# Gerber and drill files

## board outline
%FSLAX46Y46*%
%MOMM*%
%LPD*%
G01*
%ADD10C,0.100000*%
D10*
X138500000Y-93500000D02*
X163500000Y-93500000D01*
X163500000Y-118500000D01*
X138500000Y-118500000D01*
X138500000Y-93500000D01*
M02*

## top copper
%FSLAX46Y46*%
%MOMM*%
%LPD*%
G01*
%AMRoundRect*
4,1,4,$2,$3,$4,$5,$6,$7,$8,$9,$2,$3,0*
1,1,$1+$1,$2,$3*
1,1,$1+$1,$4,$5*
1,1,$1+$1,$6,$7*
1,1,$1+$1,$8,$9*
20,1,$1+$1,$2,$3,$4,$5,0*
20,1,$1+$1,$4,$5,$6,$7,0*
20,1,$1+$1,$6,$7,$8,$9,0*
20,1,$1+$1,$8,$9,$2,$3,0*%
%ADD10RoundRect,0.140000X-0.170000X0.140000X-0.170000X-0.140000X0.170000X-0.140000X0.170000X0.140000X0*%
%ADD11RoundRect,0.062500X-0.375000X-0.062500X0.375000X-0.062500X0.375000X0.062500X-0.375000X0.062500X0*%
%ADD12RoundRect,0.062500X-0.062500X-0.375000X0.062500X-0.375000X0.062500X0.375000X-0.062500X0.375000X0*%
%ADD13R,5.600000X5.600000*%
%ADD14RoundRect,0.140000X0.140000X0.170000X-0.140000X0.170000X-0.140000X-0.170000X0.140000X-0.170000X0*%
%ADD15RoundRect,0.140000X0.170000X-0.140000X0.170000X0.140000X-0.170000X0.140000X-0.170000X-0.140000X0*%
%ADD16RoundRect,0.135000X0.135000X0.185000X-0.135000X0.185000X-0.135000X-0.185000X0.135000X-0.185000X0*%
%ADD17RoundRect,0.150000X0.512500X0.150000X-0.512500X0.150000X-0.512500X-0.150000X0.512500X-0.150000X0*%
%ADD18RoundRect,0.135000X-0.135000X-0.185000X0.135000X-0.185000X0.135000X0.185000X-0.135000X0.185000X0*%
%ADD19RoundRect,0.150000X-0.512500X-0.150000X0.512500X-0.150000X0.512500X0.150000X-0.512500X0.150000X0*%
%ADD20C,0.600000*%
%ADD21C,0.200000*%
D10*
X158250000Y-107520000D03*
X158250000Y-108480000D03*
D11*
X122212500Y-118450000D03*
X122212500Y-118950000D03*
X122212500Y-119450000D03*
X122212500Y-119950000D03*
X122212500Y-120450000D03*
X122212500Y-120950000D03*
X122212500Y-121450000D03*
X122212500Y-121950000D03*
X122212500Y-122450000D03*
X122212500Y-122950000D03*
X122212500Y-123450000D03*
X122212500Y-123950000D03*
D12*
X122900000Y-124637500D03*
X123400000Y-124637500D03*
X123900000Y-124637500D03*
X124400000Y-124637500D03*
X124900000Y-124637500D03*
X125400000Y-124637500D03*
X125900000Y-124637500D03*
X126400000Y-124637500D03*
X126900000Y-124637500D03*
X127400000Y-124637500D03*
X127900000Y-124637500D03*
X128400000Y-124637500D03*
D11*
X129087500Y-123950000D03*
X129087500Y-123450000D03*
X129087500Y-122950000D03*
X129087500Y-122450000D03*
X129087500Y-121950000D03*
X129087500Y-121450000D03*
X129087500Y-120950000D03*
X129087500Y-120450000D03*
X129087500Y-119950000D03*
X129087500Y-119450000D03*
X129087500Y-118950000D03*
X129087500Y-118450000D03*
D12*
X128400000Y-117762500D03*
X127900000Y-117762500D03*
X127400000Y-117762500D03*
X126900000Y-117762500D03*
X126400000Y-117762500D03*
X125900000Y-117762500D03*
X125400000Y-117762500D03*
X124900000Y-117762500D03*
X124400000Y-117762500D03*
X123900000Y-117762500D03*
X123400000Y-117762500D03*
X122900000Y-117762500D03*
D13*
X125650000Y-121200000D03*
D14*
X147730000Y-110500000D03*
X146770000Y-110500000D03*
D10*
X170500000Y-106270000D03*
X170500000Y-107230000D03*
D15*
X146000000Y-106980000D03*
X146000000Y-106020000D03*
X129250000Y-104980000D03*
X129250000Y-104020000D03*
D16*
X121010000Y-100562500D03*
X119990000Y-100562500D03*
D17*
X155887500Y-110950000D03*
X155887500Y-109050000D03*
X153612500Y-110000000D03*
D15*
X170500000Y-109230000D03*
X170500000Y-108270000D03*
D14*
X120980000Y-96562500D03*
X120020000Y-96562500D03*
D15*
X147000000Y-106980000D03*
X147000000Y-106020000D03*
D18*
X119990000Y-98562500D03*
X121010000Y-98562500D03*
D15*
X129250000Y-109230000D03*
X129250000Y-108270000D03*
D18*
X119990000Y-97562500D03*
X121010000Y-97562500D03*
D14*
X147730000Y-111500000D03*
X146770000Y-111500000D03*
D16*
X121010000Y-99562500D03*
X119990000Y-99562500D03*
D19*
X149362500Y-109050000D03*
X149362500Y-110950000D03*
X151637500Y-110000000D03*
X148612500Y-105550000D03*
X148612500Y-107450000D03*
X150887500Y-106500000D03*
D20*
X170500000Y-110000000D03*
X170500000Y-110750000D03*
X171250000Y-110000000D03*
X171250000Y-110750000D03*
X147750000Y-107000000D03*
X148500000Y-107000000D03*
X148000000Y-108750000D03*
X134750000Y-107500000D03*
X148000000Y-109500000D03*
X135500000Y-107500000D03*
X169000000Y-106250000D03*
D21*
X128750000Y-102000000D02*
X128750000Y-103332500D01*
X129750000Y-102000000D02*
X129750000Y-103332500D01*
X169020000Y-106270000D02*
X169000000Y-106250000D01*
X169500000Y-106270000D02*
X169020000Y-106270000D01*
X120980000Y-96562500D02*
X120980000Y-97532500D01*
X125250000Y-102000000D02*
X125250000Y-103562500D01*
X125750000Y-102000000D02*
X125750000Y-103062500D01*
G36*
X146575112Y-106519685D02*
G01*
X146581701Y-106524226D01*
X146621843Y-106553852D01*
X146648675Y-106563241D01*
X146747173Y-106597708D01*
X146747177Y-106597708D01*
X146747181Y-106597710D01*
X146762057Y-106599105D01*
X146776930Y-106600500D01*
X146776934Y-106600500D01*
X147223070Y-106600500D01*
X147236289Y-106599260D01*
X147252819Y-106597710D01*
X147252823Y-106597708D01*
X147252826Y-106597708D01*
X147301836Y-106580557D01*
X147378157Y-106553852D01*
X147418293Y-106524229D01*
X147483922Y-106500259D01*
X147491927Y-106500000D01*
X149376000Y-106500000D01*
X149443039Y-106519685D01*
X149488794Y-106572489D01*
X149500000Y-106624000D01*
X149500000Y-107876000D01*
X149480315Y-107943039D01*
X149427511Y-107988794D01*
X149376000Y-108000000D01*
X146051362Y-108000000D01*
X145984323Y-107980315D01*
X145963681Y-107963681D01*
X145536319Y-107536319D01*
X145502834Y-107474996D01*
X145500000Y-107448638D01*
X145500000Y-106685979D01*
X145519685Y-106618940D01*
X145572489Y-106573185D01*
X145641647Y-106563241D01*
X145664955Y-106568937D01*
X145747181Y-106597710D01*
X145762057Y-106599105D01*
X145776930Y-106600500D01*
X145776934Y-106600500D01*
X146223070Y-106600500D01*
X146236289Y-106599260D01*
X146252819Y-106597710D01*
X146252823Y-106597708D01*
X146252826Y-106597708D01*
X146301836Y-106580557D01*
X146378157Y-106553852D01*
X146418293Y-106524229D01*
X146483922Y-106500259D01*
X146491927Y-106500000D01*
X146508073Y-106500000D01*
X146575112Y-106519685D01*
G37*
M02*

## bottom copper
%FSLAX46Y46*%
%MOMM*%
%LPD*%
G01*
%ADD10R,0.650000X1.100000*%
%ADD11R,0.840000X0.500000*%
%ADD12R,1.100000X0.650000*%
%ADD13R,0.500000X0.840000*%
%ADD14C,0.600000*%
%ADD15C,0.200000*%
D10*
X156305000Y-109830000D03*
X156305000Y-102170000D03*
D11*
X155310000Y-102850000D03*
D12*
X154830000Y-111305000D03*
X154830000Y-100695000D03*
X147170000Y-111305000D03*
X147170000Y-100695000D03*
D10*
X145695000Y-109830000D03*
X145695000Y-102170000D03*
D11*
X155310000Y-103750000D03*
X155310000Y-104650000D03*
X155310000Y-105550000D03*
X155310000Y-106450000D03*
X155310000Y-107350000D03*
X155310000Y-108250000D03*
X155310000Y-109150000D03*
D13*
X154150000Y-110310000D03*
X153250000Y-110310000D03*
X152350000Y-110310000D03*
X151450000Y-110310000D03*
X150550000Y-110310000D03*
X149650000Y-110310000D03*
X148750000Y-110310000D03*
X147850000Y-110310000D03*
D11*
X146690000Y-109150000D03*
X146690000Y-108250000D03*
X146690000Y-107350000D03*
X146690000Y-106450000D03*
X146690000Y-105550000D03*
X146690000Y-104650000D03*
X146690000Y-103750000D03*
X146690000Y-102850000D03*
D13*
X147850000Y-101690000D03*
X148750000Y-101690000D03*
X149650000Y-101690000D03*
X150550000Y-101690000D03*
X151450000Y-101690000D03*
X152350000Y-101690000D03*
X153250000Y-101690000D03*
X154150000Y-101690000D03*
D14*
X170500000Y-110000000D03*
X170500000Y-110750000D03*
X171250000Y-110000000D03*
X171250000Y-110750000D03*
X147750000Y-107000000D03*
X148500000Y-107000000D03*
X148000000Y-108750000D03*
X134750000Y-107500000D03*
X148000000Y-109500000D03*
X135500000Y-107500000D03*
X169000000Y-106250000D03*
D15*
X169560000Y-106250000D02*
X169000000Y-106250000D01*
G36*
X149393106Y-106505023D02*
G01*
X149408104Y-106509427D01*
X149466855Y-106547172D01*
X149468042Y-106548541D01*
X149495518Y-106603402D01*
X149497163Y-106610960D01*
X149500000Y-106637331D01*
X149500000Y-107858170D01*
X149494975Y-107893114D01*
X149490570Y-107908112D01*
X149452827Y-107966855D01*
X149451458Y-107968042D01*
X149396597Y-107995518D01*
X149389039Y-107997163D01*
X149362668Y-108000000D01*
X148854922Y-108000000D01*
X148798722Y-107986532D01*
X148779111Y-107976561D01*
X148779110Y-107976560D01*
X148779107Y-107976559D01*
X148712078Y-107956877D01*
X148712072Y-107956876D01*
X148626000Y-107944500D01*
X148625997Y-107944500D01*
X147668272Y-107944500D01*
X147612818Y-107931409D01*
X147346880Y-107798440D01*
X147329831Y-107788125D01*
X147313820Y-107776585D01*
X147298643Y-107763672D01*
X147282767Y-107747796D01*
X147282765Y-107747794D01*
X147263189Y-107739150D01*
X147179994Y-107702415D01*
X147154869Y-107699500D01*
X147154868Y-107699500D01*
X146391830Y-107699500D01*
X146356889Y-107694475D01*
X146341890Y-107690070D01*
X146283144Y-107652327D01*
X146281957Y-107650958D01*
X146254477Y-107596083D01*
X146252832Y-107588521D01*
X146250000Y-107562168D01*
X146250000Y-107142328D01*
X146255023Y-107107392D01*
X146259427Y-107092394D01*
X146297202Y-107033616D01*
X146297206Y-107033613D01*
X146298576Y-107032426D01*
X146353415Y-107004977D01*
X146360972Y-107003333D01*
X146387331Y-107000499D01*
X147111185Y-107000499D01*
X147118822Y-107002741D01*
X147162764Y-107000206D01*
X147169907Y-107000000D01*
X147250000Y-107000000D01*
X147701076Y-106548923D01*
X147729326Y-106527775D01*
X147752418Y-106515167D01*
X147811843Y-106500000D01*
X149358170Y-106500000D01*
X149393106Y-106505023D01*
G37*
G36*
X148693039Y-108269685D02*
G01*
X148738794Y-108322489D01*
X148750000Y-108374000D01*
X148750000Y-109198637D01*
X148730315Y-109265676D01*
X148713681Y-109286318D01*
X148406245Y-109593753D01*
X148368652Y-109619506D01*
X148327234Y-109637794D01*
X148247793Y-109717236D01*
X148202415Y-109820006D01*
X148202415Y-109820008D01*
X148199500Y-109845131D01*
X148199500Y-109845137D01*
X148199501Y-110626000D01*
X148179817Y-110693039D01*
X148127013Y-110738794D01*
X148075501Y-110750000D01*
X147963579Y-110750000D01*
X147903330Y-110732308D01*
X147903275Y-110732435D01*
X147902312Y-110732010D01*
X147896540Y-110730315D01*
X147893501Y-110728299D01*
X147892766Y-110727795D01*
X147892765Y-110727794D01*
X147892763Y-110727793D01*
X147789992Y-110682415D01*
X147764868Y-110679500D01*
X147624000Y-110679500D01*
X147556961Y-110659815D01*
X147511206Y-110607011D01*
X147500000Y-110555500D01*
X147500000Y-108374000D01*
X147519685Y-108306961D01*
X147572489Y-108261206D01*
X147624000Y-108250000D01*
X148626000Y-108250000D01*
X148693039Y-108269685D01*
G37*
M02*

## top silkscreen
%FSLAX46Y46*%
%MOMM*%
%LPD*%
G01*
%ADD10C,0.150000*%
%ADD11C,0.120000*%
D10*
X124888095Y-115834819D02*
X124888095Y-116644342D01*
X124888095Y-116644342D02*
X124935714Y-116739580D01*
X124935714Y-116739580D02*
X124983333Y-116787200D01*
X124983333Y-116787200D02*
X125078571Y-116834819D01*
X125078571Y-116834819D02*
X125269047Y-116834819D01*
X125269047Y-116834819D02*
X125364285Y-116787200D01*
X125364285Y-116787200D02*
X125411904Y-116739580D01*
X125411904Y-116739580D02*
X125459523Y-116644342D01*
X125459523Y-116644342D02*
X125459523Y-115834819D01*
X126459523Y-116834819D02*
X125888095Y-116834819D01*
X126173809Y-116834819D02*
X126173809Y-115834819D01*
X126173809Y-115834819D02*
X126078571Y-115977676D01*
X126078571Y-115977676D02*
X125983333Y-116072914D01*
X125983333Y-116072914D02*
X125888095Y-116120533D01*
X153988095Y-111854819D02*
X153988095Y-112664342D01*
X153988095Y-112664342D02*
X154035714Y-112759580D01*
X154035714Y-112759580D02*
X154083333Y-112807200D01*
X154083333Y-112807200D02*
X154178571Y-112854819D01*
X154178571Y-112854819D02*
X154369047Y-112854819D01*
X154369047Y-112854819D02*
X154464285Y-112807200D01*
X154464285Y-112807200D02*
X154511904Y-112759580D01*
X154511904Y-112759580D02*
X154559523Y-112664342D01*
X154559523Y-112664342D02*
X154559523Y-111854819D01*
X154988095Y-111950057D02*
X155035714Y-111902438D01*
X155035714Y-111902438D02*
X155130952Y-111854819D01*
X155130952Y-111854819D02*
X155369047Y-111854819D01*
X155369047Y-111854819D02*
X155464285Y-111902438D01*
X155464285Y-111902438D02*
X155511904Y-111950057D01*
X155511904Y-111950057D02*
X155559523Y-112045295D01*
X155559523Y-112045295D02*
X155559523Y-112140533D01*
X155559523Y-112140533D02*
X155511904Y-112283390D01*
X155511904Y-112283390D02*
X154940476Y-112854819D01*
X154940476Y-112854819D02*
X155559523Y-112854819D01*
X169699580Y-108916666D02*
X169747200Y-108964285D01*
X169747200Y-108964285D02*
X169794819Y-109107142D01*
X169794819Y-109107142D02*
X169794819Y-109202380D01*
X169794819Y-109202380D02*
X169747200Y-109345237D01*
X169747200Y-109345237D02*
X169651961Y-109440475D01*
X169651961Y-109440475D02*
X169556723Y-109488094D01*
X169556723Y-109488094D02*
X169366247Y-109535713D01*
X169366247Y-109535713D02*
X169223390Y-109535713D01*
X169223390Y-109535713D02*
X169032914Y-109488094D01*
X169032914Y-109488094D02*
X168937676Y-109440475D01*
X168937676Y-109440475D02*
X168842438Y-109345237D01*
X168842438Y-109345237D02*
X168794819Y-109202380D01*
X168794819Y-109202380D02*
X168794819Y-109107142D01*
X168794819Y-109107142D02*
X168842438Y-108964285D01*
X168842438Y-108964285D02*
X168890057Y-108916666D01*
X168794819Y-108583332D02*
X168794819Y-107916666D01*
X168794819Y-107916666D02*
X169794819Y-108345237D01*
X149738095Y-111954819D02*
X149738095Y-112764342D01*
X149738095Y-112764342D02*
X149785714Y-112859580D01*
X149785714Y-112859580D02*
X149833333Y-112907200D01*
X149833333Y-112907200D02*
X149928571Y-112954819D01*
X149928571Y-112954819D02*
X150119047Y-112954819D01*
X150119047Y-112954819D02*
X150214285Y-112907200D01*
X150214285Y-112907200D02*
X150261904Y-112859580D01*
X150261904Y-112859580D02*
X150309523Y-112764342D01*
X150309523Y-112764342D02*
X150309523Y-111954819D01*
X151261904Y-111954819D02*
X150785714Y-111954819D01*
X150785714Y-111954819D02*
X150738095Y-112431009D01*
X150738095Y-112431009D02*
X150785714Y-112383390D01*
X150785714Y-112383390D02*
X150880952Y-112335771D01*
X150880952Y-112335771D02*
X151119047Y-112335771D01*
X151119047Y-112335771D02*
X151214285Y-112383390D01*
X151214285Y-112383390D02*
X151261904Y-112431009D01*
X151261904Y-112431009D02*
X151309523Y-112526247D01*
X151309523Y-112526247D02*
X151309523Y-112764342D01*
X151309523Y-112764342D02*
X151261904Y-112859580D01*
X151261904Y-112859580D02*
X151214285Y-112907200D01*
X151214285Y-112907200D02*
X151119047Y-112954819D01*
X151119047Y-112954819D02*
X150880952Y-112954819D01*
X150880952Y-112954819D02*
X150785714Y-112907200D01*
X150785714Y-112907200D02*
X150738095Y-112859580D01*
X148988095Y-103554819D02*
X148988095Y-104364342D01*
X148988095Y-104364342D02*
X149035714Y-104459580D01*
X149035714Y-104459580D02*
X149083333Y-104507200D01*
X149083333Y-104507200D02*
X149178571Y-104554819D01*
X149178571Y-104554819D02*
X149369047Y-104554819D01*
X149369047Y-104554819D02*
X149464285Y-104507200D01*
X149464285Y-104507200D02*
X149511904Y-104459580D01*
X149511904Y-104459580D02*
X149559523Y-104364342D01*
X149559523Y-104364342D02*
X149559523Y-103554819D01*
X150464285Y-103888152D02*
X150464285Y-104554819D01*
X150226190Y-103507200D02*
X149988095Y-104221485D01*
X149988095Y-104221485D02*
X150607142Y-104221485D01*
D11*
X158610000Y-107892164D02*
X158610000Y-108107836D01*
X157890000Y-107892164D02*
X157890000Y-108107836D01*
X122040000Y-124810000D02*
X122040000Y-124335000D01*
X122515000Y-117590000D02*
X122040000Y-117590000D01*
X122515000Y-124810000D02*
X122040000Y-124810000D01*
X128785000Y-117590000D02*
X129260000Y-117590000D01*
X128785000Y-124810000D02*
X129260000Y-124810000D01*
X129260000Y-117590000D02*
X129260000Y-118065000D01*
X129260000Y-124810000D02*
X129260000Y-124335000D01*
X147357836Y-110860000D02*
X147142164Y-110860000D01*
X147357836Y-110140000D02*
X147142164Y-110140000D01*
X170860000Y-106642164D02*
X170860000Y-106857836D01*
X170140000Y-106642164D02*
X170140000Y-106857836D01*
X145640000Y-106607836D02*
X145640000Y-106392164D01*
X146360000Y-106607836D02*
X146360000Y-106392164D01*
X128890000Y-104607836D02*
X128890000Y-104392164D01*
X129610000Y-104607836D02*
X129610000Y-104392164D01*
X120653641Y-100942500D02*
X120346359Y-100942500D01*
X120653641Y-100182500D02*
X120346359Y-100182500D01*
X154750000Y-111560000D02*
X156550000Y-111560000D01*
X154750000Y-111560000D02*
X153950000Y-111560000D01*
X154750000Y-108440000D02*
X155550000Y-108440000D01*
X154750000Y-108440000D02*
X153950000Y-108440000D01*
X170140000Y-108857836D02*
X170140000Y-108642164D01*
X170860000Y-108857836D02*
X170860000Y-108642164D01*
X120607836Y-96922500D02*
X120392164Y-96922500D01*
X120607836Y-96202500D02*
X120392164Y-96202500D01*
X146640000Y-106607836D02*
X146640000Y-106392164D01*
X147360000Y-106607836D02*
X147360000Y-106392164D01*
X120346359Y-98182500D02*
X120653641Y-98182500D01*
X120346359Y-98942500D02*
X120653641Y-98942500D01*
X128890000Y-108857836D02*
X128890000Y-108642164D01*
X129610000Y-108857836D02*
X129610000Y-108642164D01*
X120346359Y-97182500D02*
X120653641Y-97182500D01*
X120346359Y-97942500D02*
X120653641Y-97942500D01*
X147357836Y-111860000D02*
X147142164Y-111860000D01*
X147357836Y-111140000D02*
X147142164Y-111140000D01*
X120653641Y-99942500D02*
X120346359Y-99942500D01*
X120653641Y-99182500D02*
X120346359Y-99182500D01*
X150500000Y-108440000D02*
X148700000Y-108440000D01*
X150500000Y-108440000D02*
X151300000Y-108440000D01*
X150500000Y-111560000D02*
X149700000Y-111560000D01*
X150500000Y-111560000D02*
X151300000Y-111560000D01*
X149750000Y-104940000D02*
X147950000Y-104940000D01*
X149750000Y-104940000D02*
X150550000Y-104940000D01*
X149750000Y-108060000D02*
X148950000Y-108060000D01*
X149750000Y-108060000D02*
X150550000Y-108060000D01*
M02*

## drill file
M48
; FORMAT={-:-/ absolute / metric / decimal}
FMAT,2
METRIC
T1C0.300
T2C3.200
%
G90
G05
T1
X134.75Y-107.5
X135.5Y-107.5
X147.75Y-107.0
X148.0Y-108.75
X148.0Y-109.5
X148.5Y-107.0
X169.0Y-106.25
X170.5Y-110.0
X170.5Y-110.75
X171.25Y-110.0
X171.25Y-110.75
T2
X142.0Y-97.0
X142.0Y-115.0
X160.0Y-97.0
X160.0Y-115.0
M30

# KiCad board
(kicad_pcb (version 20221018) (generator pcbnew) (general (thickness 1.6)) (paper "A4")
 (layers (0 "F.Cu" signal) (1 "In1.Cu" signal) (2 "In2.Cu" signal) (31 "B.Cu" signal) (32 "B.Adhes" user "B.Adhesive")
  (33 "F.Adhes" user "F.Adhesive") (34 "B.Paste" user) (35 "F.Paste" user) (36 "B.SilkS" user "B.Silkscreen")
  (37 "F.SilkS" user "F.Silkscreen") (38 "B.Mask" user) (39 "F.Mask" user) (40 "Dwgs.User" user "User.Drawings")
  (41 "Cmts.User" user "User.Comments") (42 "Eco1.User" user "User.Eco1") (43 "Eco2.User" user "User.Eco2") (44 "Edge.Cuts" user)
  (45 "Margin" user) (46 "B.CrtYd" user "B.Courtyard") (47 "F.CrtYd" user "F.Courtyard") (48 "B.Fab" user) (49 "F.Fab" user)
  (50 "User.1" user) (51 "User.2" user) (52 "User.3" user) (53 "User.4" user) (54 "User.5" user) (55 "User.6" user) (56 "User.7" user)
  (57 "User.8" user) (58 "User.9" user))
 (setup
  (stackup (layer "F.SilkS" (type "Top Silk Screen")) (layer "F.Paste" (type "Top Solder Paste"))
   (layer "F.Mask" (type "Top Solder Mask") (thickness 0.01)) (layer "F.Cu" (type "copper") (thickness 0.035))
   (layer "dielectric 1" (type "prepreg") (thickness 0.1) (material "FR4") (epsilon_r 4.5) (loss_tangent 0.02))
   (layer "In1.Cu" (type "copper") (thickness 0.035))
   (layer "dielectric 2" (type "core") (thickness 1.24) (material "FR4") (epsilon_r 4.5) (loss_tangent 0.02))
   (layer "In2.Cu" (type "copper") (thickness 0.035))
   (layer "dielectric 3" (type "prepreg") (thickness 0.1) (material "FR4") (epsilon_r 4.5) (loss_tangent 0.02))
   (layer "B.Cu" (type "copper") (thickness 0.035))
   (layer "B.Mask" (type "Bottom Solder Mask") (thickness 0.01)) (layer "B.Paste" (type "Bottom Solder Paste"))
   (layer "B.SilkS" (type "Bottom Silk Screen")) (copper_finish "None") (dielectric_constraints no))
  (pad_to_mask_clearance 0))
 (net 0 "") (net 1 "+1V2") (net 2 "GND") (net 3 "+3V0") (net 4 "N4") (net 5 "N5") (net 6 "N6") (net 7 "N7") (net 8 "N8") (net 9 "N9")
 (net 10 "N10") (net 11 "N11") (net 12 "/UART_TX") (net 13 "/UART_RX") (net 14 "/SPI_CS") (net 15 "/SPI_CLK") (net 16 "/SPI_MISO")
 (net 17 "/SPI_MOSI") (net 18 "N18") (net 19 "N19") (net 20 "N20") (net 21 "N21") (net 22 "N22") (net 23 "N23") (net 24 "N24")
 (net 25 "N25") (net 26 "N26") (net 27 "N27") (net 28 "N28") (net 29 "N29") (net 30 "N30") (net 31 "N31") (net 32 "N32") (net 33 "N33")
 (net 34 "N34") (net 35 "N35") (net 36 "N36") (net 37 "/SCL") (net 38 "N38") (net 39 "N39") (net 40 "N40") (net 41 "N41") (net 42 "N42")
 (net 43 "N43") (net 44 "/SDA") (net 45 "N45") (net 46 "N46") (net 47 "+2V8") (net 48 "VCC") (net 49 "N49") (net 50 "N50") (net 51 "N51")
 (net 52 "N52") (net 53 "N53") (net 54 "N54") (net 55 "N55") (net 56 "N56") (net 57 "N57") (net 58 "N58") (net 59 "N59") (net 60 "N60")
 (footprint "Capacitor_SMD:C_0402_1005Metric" (layer "F.Cu") (at 158.25 108 -90)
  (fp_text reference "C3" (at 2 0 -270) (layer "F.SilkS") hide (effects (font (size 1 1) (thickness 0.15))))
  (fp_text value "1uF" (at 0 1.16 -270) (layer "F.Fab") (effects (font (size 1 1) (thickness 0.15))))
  (fp_line (start -0.107836 -0.36) (end 0.107836 -0.36) (stroke (width 0.12) (type solid)) (layer "F.SilkS"))
  (fp_line (start -0.107836 0.36) (end 0.107836 0.36) (stroke (width 0.12) (type solid)) (layer "F.SilkS"))
  (pad "1" smd roundrect (at -0.48 0 270) (size 0.56 0.62) (layers "F.Cu" "F.Paste" "F.Mask") (roundrect_rratio 0.25) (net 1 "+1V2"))
  (pad "2" smd roundrect (at 0.48 0 270) (size 0.56 0.62) (layers "F.Cu" "F.Paste" "F.Mask") (roundrect_rratio 0.25) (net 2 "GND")))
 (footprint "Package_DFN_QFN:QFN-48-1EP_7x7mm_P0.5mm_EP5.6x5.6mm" (layer "F.Cu") (at 125.65 121.2)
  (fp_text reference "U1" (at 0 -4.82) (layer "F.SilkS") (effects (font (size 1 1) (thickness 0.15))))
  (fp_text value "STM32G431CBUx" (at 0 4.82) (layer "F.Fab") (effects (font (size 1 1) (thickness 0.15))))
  (fp_line (start -3.61 3.61) (end -3.61 3.135) (stroke (width 0.12) (type solid)) (layer "F.SilkS"))
  (fp_line (start -3.135 -3.61) (end -3.61 -3.61) (stroke (width 0.12) (type solid)) (layer "F.SilkS"))
  (fp_line (start -3.135 3.61) (end -3.61 3.61) (stroke (width 0.12) (type solid)) (layer "F.SilkS"))
  (fp_line (start 3.135 -3.61) (end 3.61 -3.61) (stroke (width 0.12) (type solid)) (layer "F.SilkS"))
  (fp_line (start 3.135 3.61) (end 3.61 3.61) (stroke (width 0.12) (type solid)) (layer "F.SilkS"))
  (fp_line (start 3.61 -3.61) (end 3.61 -3.135) (stroke (width 0.12) (type solid)) (layer "F.SilkS"))
  (fp_line (start 3.61 3.61) (end 3.61 3.135) (stroke (width 0.12) (type solid)) (layer "F.SilkS"))
  (pad "" smd roundrect (at -2.1 -2.1) (size 1.13 1.13) (layers "F.Paste") (roundrect_rratio 0.221239))
  (pad "" smd roundrect (at -2.1 -0.7) (size 1.13 1.13) (layers "F.Paste") (roundrect_rratio 0.221239))
  (pad "" smd roundrect (at -2.1 0.7) (size 1.13 1.13) (layers "F.Paste") (roundrect_rratio 0.221239))
  (pad "" smd roundrect (at -2.1 2.1) (size 1.13 1.13) (layers "F.Paste") (roundrect_rratio 0.221239))
  (pad "" smd roundrect (at -0.7 -2.1) (size 1.13 1.13) (layers "F.Paste") (roundrect_rratio 0.221239))
  (pad "" smd roundrect (at -0.7 -0.7) (size 1.13 1.13) (layers "F.Paste") (roundrect_rratio 0.221239))
  (pad "" smd roundrect (at -0.7 0.7) (size 1.13 1.13) (layers "F.Paste") (roundrect_rratio 0.221239))
  (pad "" smd roundrect (at -0.7 2.1) (size 1.13 1.13) (layers "F.Paste") (roundrect_rratio 0.221239))
  (pad "" smd roundrect (at 0.7 -2.1) (size 1.13 1.13) (layers "F.Paste") (roundrect_rratio 0.221239))
  (pad "" smd roundrect (at 0.7 -0.7) (size 1.13 1.13) (layers "F.Paste") (roundrect_rratio 0.221239))
  (pad "" smd roundrect (at 0.7 0.7) (size 1.13 1.13) (layers "F.Paste") (roundrect_rratio 0.221239))
  (pad "" smd roundrect (at 0.7 2.1) (size 1.13 1.13) (layers "F.Paste") (roundrect_rratio 0.221239))
  (pad "" smd roundrect (at 2.1 -2.1) (size 1.13 1.13) (layers "F.Paste") (roundrect_rratio 0.221239))
  (pad "" smd roundrect (at 2.1 -0.7) (size 1.13 1.13) (layers "F.Paste") (roundrect_rratio 0.221239))
  (pad "" smd roundrect (at 2.1 0.7) (size 1.13 1.13) (layers "F.Paste") (roundrect_rratio 0.221239))
  (pad "" smd roundrect (at 2.1 2.1) (size 1.13 1.13) (layers "F.Paste") (roundrect_rratio 0.221239))
  (pad "1" smd roundrect (at -3.4375 -2.75) (size 0.875 0.25) (layers "F.Cu" "F.Paste" "F.Mask") (roundrect_rratio 0.25) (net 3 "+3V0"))
  (pad "2" smd roundrect (at -3.4375 -2.25) (size 0.875 0.25) (layers "F.Cu" "F.Paste" "F.Mask") (roundrect_rratio 0.25) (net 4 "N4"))
  (pad "3" smd roundrect (at -3.4375 -1.75) (size 0.875 0.25) (layers "F.Cu" "F.Paste" "F.Mask") (roundrect_rratio 0.25) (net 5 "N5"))
  (pad "4" smd roundrect (at -3.4375 -1.25) (size 0.875 0.25) (layers "F.Cu" "F.Paste" "F.Mask") (roundrect_rratio 0.25) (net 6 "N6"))
  (pad "5" smd roundrect (at -3.4375 -0.75) (size 0.875 0.25) (layers "F.Cu" "F.Paste" "F.Mask") (roundrect_rratio 0.25) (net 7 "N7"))
  (pad "6" smd roundrect (at -3.4375 -0.25) (size 0.875 0.25) (layers "F.Cu" "F.Paste" "F.Mask") (roundrect_rratio 0.25) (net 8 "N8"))
  (pad "7" smd roundrect (at -3.4375 0.25) (size 0.875 0.25) (layers "F.Cu" "F.Paste" "F.Mask") (roundrect_rratio 0.25) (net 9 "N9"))
  (pad "8" smd roundrect (at -3.4375 0.75) (size 0.875 0.25) (layers "F.Cu" "F.Paste" "F.Mask") (roundrect_rratio 0.25) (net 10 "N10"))
  (pad "9" smd roundrect (at -3.4375 1.25) (size 0.875 0.25) (layers "F.Cu" "F.Paste" "F.Mask") (roundrect_rratio 0.25) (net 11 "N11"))
  (pad "10" smd roundrect (at -3.4375 1.75) (size 0.875 0.25) (layers "F.Cu" "F.Paste" "F.Mask") (roundrect_rratio 0.25) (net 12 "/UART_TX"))
  (pad "11" smd roundrect (at -3.4375 2.25) (size 0.875 0.25) (layers "F.Cu" "F.Paste" "F.Mask") (roundrect_rratio 0.25) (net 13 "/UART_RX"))
  (pad "12" smd roundrect (at -3.4375 2.75) (size 0.875 0.25) (layers "F.Cu" "F.Paste" "F.Mask") (roundrect_rratio 0.25) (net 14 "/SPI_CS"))
  (pad "13" smd roundrect (at -2.75 3.4375) (size 0.25 0.875) (layers "F.Cu" "F.Paste" "F.Mask") (roundrect_rratio 0.25) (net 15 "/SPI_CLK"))
  (pad "14" smd roundrect (at -2.25 3.4375) (size 0.25 0.875) (layers "F.Cu" "F.Paste" "F.Mask") (roundrect_rratio 0.25)
   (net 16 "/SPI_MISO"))
  (pad "15" smd roundrect (at -1.75 3.4375) (size 0.25 0.875) (layers "F.Cu" "F.Paste" "F.Mask") (roundrect_rratio 0.25)
   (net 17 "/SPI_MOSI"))
  (pad "16" smd roundrect (at -1.25 3.4375) (size 0.25 0.875) (layers "F.Cu" "F.Paste" "F.Mask") (roundrect_rratio 0.25) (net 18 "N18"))
  (pad "17" smd roundrect (at -0.75 3.4375) (size 0.25 0.875) (layers "F.Cu" "F.Paste" "F.Mask") (roundrect_rratio 0.25) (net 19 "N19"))
  (pad "18" smd roundrect (at -0.25 3.4375) (size 0.25 0.875) (layers "F.Cu" "F.Paste" "F.Mask") (roundrect_rratio 0.25) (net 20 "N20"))
  (pad "19" smd roundrect (at 0.25 3.4375) (size 0.25 0.875) (layers "F.Cu" "F.Paste" "F.Mask") (roundrect_rratio 0.25) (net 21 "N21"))
  (pad "20" smd roundrect (at 0.75 3.4375) (size 0.25 0.875) (layers "F.Cu" "F.Paste" "F.Mask") (roundrect_rratio 0.25) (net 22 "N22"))
  (pad "21" smd roundrect (at 1.25 3.4375) (size 0.25 0.875) (layers "F.Cu" "F.Paste" "F.Mask") (roundrect_rratio 0.25) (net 3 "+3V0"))
  (pad "22" smd roundrect (at 1.75 3.4375) (size 0.25 0.875) (layers "F.Cu" "F.Paste" "F.Mask") (roundrect_rratio 0.25) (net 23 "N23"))
  (pad "23" smd roundrect (at 2.25 3.4375) (size 0.25 0.875) (layers "F.Cu" "F.Paste" "F.Mask") (roundrect_rratio 0.25) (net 3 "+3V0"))
  (pad "24" smd roundrect (at 2.75 3.4375) (size 0.25 0.875) (layers "F.Cu" "F.Paste" "F.Mask") (roundrect_rratio 0.25) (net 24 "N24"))
  (pad "25" smd roundrect (at 3.4375 2.75) (size 0.875 0.25) (layers "F.Cu" "F.Paste" "F.Mask") (roundrect_rratio 0.25) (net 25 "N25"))
  (pad "26" smd roundrect (at 3.4375 2.25) (size 0.875 0.25) (layers "F.Cu" "F.Paste" "F.Mask") (roundrect_rratio 0.25) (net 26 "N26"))
  (pad "27" smd roundrect (at 3.4375 1.75) (size 0.875 0.25) (layers "F.Cu" "F.Paste" "F.Mask") (roundrect_rratio 0.25) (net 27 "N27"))
  (pad "28" smd roundrect (at 3.4375 1.25) (size 0.875 0.25) (layers "F.Cu" "F.Paste" "F.Mask") (roundrect_rratio 0.25) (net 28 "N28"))
  (pad "29" smd roundrect (at 3.4375 0.75) (size 0.875 0.25) (layers "F.Cu" "F.Paste" "F.Mask") (roundrect_rratio 0.25) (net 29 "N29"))
  (pad "30" smd roundrect (at 3.4375 0.25) (size 0.875 0.25) (layers "F.Cu" "F.Paste" "F.Mask") (roundrect_rratio 0.25) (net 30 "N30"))
  (pad "31" smd roundrect (at 3.4375 -0.25) (size 0.875 0.25) (layers "F.Cu" "F.Paste" "F.Mask") (roundrect_rratio 0.25) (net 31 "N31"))
  (pad "32" smd roundrect (at 3.4375 -0.75) (size 0.875 0.25) (layers "F.Cu" "F.Paste" "F.Mask") (roundrect_rratio 0.25) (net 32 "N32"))
  (pad "33" smd roundrect (at 3.4375 -1.25) (size 0.875 0.25) (layers "F.Cu" "F.Paste" "F.Mask") (roundrect_rratio 0.25) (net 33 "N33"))
  (pad "34" smd roundrect (at 3.4375 -1.75) (size 0.875 0.25) (layers "F.Cu" "F.Paste" "F.Mask") (roundrect_rratio 0.25) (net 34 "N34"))
  (pad "35" smd roundrect (at 3.4375 -2.25) (size 0.875 0.25) (layers "F.Cu" "F.Paste" "F.Mask") (roundrect_rratio 0.25) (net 3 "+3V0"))
  (pad "36" smd roundrect (at 3.4375 -2.75) (size 0.875 0.25) (layers "F.Cu" "F.Paste" "F.Mask") (roundrect_rratio 0.25) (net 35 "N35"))
  (pad "37" smd roundrect (at 2.75 -3.4375) (size 0.25 0.875) (layers "F.Cu" "F.Paste" "F.Mask") (roundrect_rratio 0.25) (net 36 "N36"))
  (pad "38" smd roundrect (at 2.25 -3.4375) (size 0.25 0.875) (layers "F.Cu" "F.Paste" "F.Mask") (roundrect_rratio 0.25) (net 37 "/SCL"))
  (pad "39" smd roundrect (at 1.75 -3.4375) (size 0.25 0.875) (layers "F.Cu" "F.Paste" "F.Mask") (roundrect_rratio 0.25) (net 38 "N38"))
  (pad "40" smd roundrect (at 1.25 -3.4375) (size 0.25 0.875) (layers "F.Cu" "F.Paste" "F.Mask") (roundrect_rratio 0.25) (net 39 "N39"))
  (pad "41" smd roundrect (at 0.75 -3.4375) (size 0.25 0.875) (layers "F.Cu" "F.Paste" "F.Mask") (roundrect_rratio 0.25) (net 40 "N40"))
  (pad "42" smd roundrect (at 0.25 -3.4375) (size 0.25 0.875) (layers "F.Cu" "F.Paste" "F.Mask") (roundrect_rratio 0.25) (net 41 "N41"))
  (pad "43" smd roundrect (at -0.25 -3.4375) (size 0.25 0.875) (layers "F.Cu" "F.Paste" "F.Mask") (roundrect_rratio 0.25) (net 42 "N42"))
  (pad "44" smd roundrect (at -0.75 -3.4375) (size 0.25 0.875) (layers "F.Cu" "F.Paste" "F.Mask") (roundrect_rratio 0.25) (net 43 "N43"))
  (pad "45" smd roundrect (at -1.25 -3.4375) (size 0.25 0.875) (layers "F.Cu" "F.Paste" "F.Mask") (roundrect_rratio 0.25) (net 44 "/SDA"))
  (pad "46" smd roundrect (at -1.75 -3.4375) (size 0.25 0.875) (layers "F.Cu" "F.Paste" "F.Mask") (roundrect_rratio 0.25) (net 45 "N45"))
  (pad "47" smd roundrect (at -2.25 -3.4375) (size 0.25 0.875) (layers "F.Cu" "F.Paste" "F.Mask") (roundrect_rratio 0.25) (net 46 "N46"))
  (pad "48" smd roundrect (at -2.75 -3.4375) (size 0.25 0.875) (layers "F.Cu" "F.Paste" "F.Mask") (roundrect_rratio 0.25) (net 3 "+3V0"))
  (pad "49" smd rect (at 0 0) (size 5.6 5.6) (layers "F.Cu" "F.Mask") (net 2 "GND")))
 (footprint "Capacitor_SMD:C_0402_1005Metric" (layer "F.Cu") (at 147.25 110.5 180)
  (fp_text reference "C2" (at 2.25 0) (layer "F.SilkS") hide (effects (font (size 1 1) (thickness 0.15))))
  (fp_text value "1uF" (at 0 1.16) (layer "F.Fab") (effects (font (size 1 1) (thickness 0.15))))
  (fp_line (start -0.107836 -0.36) (end 0.107836 -0.36) (stroke (width 0.12) (type solid)) (layer "F.SilkS"))
  (fp_line (start -0.107836 0.36) (end 0.107836 0.36) (stroke (width 0.12) (type solid)) (layer "F.SilkS"))
  (pad "1" smd roundrect (at -0.48 0 180) (size 0.56 0.62) (layers "F.Cu" "F.Paste" "F.Mask") (roundrect_rratio 0.25) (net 3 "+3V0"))
  (pad "2" smd roundrect (at 0.48 0 180) (size 0.56 0.62) (layers "F.Cu" "F.Paste" "F.Mask") (roundrect_rratio 0.25) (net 2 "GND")))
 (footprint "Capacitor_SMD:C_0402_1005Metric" (layer "F.Cu") (at 170.5 106.75 -90)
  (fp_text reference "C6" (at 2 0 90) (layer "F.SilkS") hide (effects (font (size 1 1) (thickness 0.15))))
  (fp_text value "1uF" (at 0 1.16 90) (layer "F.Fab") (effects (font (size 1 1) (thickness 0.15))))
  (fp_line (start -0.107836 -0.36) (end 0.107836 -0.36) (stroke (width 0.12) (type solid)) (layer "F.SilkS"))
  (fp_line (start -0.107836 0.36) (end 0.107836 0.36) (stroke (width 0.12) (type solid)) (layer "F.SilkS"))
  (pad "1" smd roundrect (at -0.48 0 270) (size 0.56 0.62) (layers "F.Cu" "F.Paste" "F.Mask") (roundrect_rratio 0.25) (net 1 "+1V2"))
  (pad "2" smd roundrect (at 0.48 0 270) (size 0.56 0.62) (layers "F.Cu" "F.Paste" "F.Mask") (roundrect_rratio 0.25) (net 2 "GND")))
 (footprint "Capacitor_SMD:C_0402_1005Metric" (layer "F.Cu") (at 146 106.5 90)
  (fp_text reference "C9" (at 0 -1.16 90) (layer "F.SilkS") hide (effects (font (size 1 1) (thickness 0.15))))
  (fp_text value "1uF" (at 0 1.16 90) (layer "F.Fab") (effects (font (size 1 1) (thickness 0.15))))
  (fp_line (start -0.107836 -0.36) (end 0.107836 -0.36) (stroke (width 0.12) (type solid)) (layer "F.SilkS"))
  (fp_line (start -0.107836 0.36) (end 0.107836 0.36) (stroke (width 0.12) (type solid)) (layer "F.SilkS"))
  (pad "1" smd roundrect (at -0.48 0 90) (size 0.56 0.62) (layers "F.Cu" "F.Paste" "F.Mask") (roundrect_rratio 0.25) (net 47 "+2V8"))
  (pad "2" smd roundrect (at 0.48 0 90) (size 0.56 0.62) (layers "F.Cu" "F.Paste" "F.Mask") (roundrect_rratio 0.25) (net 2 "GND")))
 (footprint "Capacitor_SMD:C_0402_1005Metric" (layer "F.Cu") (at 129.25 104.5 90)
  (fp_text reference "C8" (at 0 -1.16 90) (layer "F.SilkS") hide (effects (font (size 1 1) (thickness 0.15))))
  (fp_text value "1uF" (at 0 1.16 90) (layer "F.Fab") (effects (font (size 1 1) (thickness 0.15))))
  (fp_line (start -0.107836 -0.36) (end 0.107836 -0.36) (stroke (width 0.12) (type solid)) (layer "F.SilkS"))
  (fp_line (start -0.107836 0.36) (end 0.107836 0.36) (stroke (width 0.12) (type solid)) (layer "F.SilkS"))
  (pad "1" smd roundrect (at -0.48 0 90) (size 0.56 0.62) (layers "F.Cu" "F.Paste" "F.Mask") (roundrect_rratio 0.25) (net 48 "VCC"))
  (pad "2" smd roundrect (at 0.48 0 90) (size 0.56 0.62) (layers "F.Cu" "F.Paste" "F.Mask") (roundrect_rratio 0.25) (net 2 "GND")))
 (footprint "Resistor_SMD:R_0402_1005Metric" (layer "F.Cu") (at 120.5 100.5625 180)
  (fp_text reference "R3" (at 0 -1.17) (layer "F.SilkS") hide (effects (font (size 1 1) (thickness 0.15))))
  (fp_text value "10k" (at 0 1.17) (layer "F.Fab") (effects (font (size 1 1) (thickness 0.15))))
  (fp_line (start -0.153641 -0.38) (end 0.153641 -0.38) (stroke (width 0.12) (type solid)) (layer "F.SilkS"))
  (fp_line (start -0.153641 0.38) (end 0.153641 0.38) (stroke (width 0.12) (type solid)) (layer "F.SilkS"))
  (pad "1" smd roundrect (at -0.51 0 180) (size 0.54 0.64) (layers "F.Cu" "F.Paste" "F.Mask") (roundrect_rratio 0.25) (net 37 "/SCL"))
  (pad "2" smd roundrect (at 0.51 0 180) (size 0.54 0.64) (layers "F.Cu" "F.Paste" "F.Mask") (roundrect_rratio 0.25) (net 3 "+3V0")))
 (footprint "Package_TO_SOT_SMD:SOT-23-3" (layer "F.Cu") (at 154.75 110 180)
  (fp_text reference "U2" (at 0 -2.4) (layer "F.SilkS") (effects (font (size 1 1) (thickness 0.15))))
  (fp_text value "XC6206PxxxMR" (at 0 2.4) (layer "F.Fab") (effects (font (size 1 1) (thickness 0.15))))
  (fp_line (start 0 -1.56) (end -1.8 -1.56) (stroke (width 0.12) (type solid)) (layer "F.SilkS"))
  (fp_line (start 0 -1.56) (end 0.8 -1.56) (stroke (width 0.12) (type solid)) (layer "F.SilkS"))
  (fp_line (start 0 1.56) (end -0.8 1.56) (stroke (width 0.12) (type solid)) (layer "F.SilkS"))
  (fp_line (start 0 1.56) (end 0.8 1.56) (stroke (width 0.12) (type solid)) (layer "F.SilkS"))
  (pad "1" smd roundrect (at -1.1375 -0.95 180) (size 1.325 0.6) (layers "F.Cu" "F.Paste" "F.Mask") (roundrect_rratio 0.25) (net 2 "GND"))
  (pad "2" smd roundrect (at -1.1375 0.95 180) (size 1.325 0.6) (layers "F.Cu" "F.Paste" "F.Mask") (roundrect_rratio 0.25) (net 1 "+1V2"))
  (pad "3" smd roundrect (at 1.1375 0 180) (size 1.325 0.6) (layers "F.Cu" "F.Paste" "F.Mask") (roundrect_rratio 0.25) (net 48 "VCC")))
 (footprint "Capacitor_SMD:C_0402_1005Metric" (layer "F.Cu") (at 170.5 108.75 90)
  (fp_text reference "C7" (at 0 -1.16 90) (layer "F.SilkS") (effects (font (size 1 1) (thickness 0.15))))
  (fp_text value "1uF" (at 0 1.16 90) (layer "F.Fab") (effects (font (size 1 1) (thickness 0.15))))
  (fp_line (start -0.107836 -0.36) (end 0.107836 -0.36) (stroke (width 0.12) (type solid)) (layer "F.SilkS"))
  (fp_line (start -0.107836 0.36) (end 0.107836 0.36) (stroke (width 0.12) (type solid)) (layer "F.SilkS"))
  (pad "1" smd roundrect (at -0.48 0 90) (size 0.56 0.62) (layers "F.Cu" "F.Paste" "F.Mask") (roundrect_rratio 0.25) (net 48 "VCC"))
  (pad "2" smd roundrect (at 0.48 0 90) (size 0.56 0.62) (layers "F.Cu" "F.Paste" "F.Mask") (roundrect_rratio 0.25) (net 2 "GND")))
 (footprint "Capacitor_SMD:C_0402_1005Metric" (layer "F.Cu") (at 120.5 96.5625 180)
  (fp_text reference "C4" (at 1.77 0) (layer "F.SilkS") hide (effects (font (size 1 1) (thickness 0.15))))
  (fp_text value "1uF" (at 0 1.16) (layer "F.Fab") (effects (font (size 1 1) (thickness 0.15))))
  (fp_line (start -0.107836 -0.36) (end 0.107836 -0.36) (stroke (width 0.12) (type solid)) (layer "F.SilkS"))
  (fp_line (start -0.107836 0.36) (end 0.107836 0.36) (stroke (width 0.12) (type solid)) (layer "F.SilkS"))
  (pad "1" smd roundrect (at -0.48 0 180) (size 0.56 0.62) (layers "F.Cu" "F.Paste" "F.Mask") (roundrect_rratio 0.25) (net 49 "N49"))
  (pad "2" smd roundrect (at 0.48 0 180) (size 0.56 0.62) (layers "F.Cu" "F.Paste" "F.Mask") (roundrect_rratio 0.25) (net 2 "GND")))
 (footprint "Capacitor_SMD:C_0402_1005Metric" (layer "F.Cu") (at 147 106.5 90)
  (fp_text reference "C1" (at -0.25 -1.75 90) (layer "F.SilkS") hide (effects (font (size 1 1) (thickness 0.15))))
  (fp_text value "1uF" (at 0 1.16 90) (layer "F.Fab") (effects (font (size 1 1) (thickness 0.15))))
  (fp_line (start -0.107836 -0.36) (end 0.107836 -0.36) (stroke (width 0.12) (type solid)) (layer "F.SilkS"))
  (fp_line (start -0.107836 0.36) (end 0.107836 0.36) (stroke (width 0.12) (type solid)) (layer "F.SilkS"))
  (pad "1" smd roundrect (at -0.48 0 90) (size 0.56 0.62) (layers "F.Cu" "F.Paste" "F.Mask") (roundrect_rratio 0.25) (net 47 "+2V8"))
  (pad "2" smd roundrect (at 0.48 0 90) (size 0.56 0.62) (layers "F.Cu" "F.Paste" "F.Mask") (roundrect_rratio 0.25) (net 2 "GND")))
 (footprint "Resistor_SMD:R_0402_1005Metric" (layer "F.Cu") (at 120.5 98.5625)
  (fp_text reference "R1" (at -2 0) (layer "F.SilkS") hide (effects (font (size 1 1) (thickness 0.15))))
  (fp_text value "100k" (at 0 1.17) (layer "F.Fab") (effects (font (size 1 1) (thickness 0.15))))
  (fp_line (start -0.153641 -0.38) (end 0.153641 -0.38) (stroke (width 0.12) (type solid)) (layer "F.SilkS"))
  (fp_line (start -0.153641 0.38) (end 0.153641 0.38) (stroke (width 0.12) (type solid)) (layer "F.SilkS"))
  (pad "1" smd roundrect (at -0.51 0) (size 0.54 0.64) (layers "F.Cu" "F.Paste" "F.Mask") (roundrect_rratio 0.25) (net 3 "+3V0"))
  (pad "2" smd roundrect (at 0.51 0) (size 0.54 0.64) (layers "F.Cu" "F.Paste" "F.Mask") (roundrect_rratio 0.25) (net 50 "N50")))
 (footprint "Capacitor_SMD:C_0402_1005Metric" (layer "F.Cu") (at 129.25 108.75 90)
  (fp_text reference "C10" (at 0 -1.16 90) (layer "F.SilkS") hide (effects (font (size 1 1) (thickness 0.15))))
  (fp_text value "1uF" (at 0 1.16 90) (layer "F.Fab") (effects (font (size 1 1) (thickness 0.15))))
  (fp_line (start -0.107836 -0.36) (end 0.107836 -0.36) (stroke (width 0.12) (type solid)) (layer "F.SilkS"))
  (fp_line (start -0.107836 0.36) (end 0.107836 0.36) (stroke (width 0.12) (type solid)) (layer "F.SilkS"))
  (pad "1" smd roundrect (at -0.48 0 90) (size 0.56 0.62) (layers "F.Cu" "F.Paste" "F.Mask") (roundrect_rratio 0.25) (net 48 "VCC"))
  (pad "2" smd roundrect (at 0.48 0 90) (size 0.56 0.62) (layers "F.Cu" "F.Paste" "F.Mask") (roundrect_rratio 0.25) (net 2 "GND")))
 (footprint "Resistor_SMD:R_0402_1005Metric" (layer "F.Cu") (at 120.5 97.5625)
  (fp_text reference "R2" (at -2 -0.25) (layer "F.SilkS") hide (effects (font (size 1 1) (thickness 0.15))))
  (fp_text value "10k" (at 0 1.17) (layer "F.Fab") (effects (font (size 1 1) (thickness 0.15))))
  (fp_line (start -0.153641 -0.38) (end 0.153641 -0.38) (stroke (width 0.12) (type solid)) (layer "F.SilkS"))
  (fp_line (start -0.153641 0.38) (end 0.153641 0.38) (stroke (width 0.12) (type solid)) (layer "F.SilkS"))
  (pad "1" smd roundrect (at -0.51 0) (size 0.54 0.64) (layers "F.Cu" "F.Paste" "F.Mask") (roundrect_rratio 0.25) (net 3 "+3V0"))
  (pad "2" smd roundrect (at 0.51 0) (size 0.54 0.64) (layers "F.Cu" "F.Paste" "F.Mask") (roundrect_rratio 0.25) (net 49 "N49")))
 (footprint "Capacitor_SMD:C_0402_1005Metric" (layer "F.Cu") (at 147.25 111.5 180)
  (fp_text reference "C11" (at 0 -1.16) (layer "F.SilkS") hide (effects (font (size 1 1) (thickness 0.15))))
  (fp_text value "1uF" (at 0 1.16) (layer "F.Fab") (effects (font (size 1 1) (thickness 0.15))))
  (fp_line (start -0.107836 -0.36) (end 0.107836 -0.36) (stroke (width 0.12) (type solid)) (layer "F.SilkS"))
  (fp_line (start -0.107836 0.36) (end 0.107836 0.36) (stroke (width 0.12) (type solid)) (layer "F.SilkS"))
  (pad "1" smd roundrect (at -0.48 0 180) (size 0.56 0.62) (layers "F.Cu" "F.Paste" "F.Mask") (roundrect_rratio 0.25) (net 3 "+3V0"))
  (pad "2" smd roundrect (at 0.48 0 180) (size 0.56 0.62) (layers "F.Cu" "F.Paste" "F.Mask") (roundrect_rratio 0.25) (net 2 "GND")))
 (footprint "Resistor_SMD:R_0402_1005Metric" (layer "F.Cu") (at 120.5 99.5625 180)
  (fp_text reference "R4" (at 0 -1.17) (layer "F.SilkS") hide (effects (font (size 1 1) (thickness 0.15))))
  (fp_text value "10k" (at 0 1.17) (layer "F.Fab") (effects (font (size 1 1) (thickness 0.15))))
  (fp_line (start -0.153641 -0.38) (end 0.153641 -0.38) (stroke (width 0.12) (type solid)) (layer "F.SilkS"))
  (fp_line (start -0.153641 0.38) (end 0.153641 0.38) (stroke (width 0.12) (type solid)) (layer "F.SilkS"))
  (pad "1" smd roundrect (at -0.51 0 180) (size 0.54 0.64) (layers "F.Cu" "F.Paste" "F.Mask") (roundrect_rratio 0.25) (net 44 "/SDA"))
  (pad "2" smd roundrect (at 0.51 0 180) (size 0.54 0.64) (layers "F.Cu" "F.Paste" "F.Mask") (roundrect_rratio 0.25) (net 3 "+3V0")))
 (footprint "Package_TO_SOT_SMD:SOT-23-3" (layer "F.Cu") (at 150.5 110)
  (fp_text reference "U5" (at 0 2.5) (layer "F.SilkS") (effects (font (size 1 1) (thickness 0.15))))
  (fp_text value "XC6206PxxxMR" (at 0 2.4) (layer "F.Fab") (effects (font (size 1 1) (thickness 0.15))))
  (fp_line (start 0 -1.56) (end -1.8 -1.56) (stroke (width 0.12) (type solid)) (layer "F.SilkS"))
  (fp_line (start 0 -1.56) (end 0.8 -1.56) (stroke (width 0.12) (type solid)) (layer "F.SilkS"))
  (fp_line (start 0 1.56) (end -0.8 1.56) (stroke (width 0.12) (type solid)) (layer "F.SilkS"))
  (fp_line (start 0 1.56) (end 0.8 1.56) (stroke (width 0.12) (type solid)) (layer "F.SilkS"))
  (pad "1" smd roundrect (at -1.1375 -0.95) (size 1.325 0.6) (layers "F.Cu" "F.Paste" "F.Mask") (roundrect_rratio 0.25) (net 2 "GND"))
  (pad "2" smd roundrect (at -1.1375 0.95) (size 1.325 0.6) (layers "F.Cu" "F.Paste" "F.Mask") (roundrect_rratio 0.25) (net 3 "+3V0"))
  (pad "3" smd roundrect (at 1.1375 0) (size 1.325 0.6) (layers "F.Cu" "F.Paste" "F.Mask") (roundrect_rratio 0.25) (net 48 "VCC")))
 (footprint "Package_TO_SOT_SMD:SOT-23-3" (layer "F.Cu") (at 149.75 106.5)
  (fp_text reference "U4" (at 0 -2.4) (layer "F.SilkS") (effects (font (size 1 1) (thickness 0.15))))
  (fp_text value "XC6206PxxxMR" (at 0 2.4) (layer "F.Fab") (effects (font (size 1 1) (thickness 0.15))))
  (fp_line (start 0 -1.56) (end -1.8 -1.56) (stroke (width 0.12) (type solid)) (layer "F.SilkS"))
  (fp_line (start 0 -1.56) (end 0.8 -1.56) (stroke (width 0.12) (type solid)) (layer "F.SilkS"))
  (fp_line (start 0 1.56) (end -0.8 1.56) (stroke (width 0.12) (type solid)) (layer "F.SilkS"))
  (fp_line (start 0 1.56) (end 0.8 1.56) (stroke (width 0.12) (type solid)) (layer "F.SilkS"))
  (pad "1" smd roundrect (at -1.1375 -0.95) (size 1.325 0.6) (layers "F.Cu" "F.Paste" "F.Mask") (roundrect_rratio 0.25) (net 2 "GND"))
  (pad "2" smd roundrect (at -1.1375 0.95) (size 1.325 0.6) (layers "F.Cu" "F.Paste" "F.Mask") (roundrect_rratio 0.25) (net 47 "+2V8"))
  (pad "3" smd roundrect (at 1.1375 0) (size 1.325 0.6) (layers "F.Cu" "F.Paste" "F.Mask") (roundrect_rratio 0.25) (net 48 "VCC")))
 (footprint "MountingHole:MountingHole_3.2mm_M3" (layer "B.Cu") (at 142 115 180)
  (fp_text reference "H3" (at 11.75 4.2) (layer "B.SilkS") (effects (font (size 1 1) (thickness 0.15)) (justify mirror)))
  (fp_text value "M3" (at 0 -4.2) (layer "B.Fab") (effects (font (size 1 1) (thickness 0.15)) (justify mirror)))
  (pad "" np_thru_hole circle (at 0 0 180) (size 3.2 3.2) (drill 3.2) (layers "*.Cu" "*.Mask")))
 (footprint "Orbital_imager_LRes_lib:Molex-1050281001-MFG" (layer "B.Cu") (at 151 106 180)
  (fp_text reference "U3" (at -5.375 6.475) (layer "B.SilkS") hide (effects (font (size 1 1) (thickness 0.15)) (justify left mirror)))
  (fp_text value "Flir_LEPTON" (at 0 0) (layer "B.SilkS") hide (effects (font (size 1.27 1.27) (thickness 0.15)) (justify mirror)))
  (pad "1" smd rect (at -5.305 -3.83 180) (size 0.65 1.1) (layers "B.Cu" "B.Paste" "B.Mask") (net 2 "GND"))
  (pad "1" smd rect (at -5.305 3.83 180) (size 0.65 1.1) (layers "B.Cu" "B.Paste" "B.Mask") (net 2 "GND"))
  (pad "1" smd rect (at -4.31 3.15 180) (size 0.84 0.5) (layers "B.Cu" "B.Paste" "B.Mask") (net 2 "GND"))
  (pad "1" smd rect (at -3.83 -5.305 180) (size 1.1 0.65) (layers "B.Cu" "B.Paste" "B.Mask") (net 2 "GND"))
  (pad "1" smd rect (at -3.83 5.305 180) (size 1.1 0.65) (layers "B.Cu" "B.Paste" "B.Mask") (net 2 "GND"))
  (pad "1" smd rect (at 3.83 -5.305 180) (size 1.1 0.65) (layers "B.Cu" "B.Paste" "B.Mask") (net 2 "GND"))
  (pad "1" smd rect (at 3.83 5.305 180) (size 1.1 0.65) (layers "B.Cu" "B.Paste" "B.Mask") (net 2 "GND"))
  (pad "1" smd rect (at 5.305 -3.83 180) (size 0.65 1.1) (layers "B.Cu" "B.Paste" "B.Mask") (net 2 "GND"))
  (pad "1" smd rect (at 5.305 3.83 180) (size 0.65 1.1) (layers "B.Cu" "B.Paste" "B.Mask") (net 2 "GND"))
  (pad "2" smd rect (at -4.31 2.25 180) (size 0.84 0.5) (layers "B.Cu" "B.Paste" "B.Mask") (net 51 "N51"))
  (pad "3" smd rect (at -4.31 1.35 180) (size 0.84 0.5) (layers "B.Cu" "B.Paste" "B.Mask") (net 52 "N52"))
  (pad "4" smd rect (at -4.31 0.45 180) (size 0.84 0.5) (layers "B.Cu" "B.Paste" "B.Mask") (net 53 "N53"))
  (pad "5" smd rect (at -4.31 -0.45 180) (size 0.84 0.5) (layers "B.Cu" "B.Paste" "B.Mask") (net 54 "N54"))
  (pad "6" smd rect (at -4.31 -1.35 180) (size 0.84 0.5) (layers "B.Cu" "B.Paste" "B.Mask") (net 2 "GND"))
  (pad "7" smd rect (at -4.31 -2.25 180) (size 0.84 0.5) (layers "B.Cu" "B.Paste" "B.Mask") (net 1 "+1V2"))
  (pad "8" smd rect (at -4.31 -3.15 180) (size 0.84 0.5) (layers "B.Cu" "B.Paste" "B.Mask") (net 2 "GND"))
  (pad "9" smd rect (at -3.15 -4.31 180) (size 0.5 0.84) (layers "B.Cu" "B.Paste" "B.Mask") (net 2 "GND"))
  (pad "10" smd rect (at -2.25 -4.31 180) (size 0.5 0.84) (layers "B.Cu" "B.Paste" "B.Mask") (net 2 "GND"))
  (pad "11" smd rect (at -1.35 -4.31 180) (size 0.5 0.84) (layers "B.Cu" "B.Paste" "B.Mask") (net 17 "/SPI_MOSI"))
  (pad "12" smd rect (at -0.45 -4.31 180) (size 0.5 0.84) (layers "B.Cu" "B.Paste" "B.Mask") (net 16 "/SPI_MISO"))
  (pad "13" smd rect (at 0.45 -4.31 180) (size 0.5 0.84) (layers "B.Cu" "B.Paste" "B.Mask") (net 15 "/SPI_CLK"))
  (pad "14" smd rect (at 1.35 -4.31 180) (size 0.5 0.84) (layers "B.Cu" "B.Paste" "B.Mask") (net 14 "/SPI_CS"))
  (pad "15" smd rect (at 2.25 -4.31 180) (size 0.5 0.84) (layers "B.Cu" "B.Paste" "B.Mask") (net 2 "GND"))
  (pad "16" smd rect (at 3.15 -4.31 180) (size 0.5 0.84) (layers "B.Cu" "B.Paste" "B.Mask") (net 3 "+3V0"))
  (pad "17" smd rect (at 4.31 -3.15 180) (size 0.84 0.5) (layers "B.Cu" "B.Paste" "B.Mask") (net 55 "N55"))
  (pad "18" smd rect (at 4.31 -2.25 180) (size 0.84 0.5) (layers "B.Cu" "B.Paste" "B.Mask") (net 2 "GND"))
  (pad "19" smd rect (at 4.31 -1.35 180) (size 0.84 0.5) (layers "B.Cu" "B.Paste" "B.Mask") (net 47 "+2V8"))
  (pad "20" smd rect (at 4.31 -0.45 180) (size 0.84 0.5) (layers "B.Cu" "B.Paste" "B.Mask") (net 2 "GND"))
  (pad "21" smd rect (at 4.31 0.45 180) (size 0.84 0.5) (layers "B.Cu" "B.Paste" "B.Mask") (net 37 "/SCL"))
  (pad "22" smd rect (at 4.31 1.35 180) (size 0.84 0.5) (layers "B.Cu" "B.Paste" "B.Mask") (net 44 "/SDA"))
  (pad "23" smd rect (at 4.31 2.25 180) (size 0.84 0.5) (layers "B.Cu" "B.Paste" "B.Mask") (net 50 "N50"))
  (pad "24" smd rect (at 4.31 3.15 180) (size 0.84 0.5) (layers "B.Cu" "B.Paste" "B.Mask") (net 49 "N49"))
  (pad "25" smd rect (at 3.15 4.31 180) (size 0.5 0.84) (layers "B.Cu" "B.Paste" "B.Mask") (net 2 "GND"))
  (pad "26" smd rect (at 2.25 4.31 180) (size 0.5 0.84) (layers "B.Cu" "B.Paste" "B.Mask") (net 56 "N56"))
  (pad "27" smd rect (at 1.35 4.31 180) (size 0.5 0.84) (layers "B.Cu" "B.Paste" "B.Mask") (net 2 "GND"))
  (pad "28" smd rect (at 0.45 4.31 180) (size 0.5 0.84) (layers "B.Cu" "B.Paste" "B.Mask") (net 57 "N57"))
  (pad "29" smd rect (at -0.45 4.31 180) (size 0.5 0.84) (layers "B.Cu" "B.Paste" "B.Mask") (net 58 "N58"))
  (pad "30" smd rect (at -1.35 4.31 180) (size 0.5 0.84) (layers "B.Cu" "B.Paste" "B.Mask") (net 2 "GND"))
  (pad "31" smd rect (at -2.25 4.31 180) (size 0.5 0.84) (layers "B.Cu" "B.Paste" "B.Mask") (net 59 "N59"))
  (pad "32" smd rect (at -3.15 4.31 180) (size 0.5 0.84) (layers "B.Cu" "B.Paste" "B.Mask") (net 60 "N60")))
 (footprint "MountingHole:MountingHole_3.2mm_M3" (layer "B.Cu") (at 142 97 180)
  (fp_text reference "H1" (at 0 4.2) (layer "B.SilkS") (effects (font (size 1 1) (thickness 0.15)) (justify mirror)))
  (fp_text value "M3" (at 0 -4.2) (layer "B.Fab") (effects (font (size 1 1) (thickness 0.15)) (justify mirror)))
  (pad "" np_thru_hole circle (at 0 0 180) (size 3.2 3.2) (drill 3.2) (layers "*.Cu" "*.Mask")))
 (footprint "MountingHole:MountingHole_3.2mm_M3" (layer "B.Cu") (at 160 115 180)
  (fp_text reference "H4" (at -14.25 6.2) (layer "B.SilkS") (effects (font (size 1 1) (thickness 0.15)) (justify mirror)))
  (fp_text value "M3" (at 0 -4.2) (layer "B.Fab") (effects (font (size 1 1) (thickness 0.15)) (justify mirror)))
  (pad "" np_thru_hole circle (at 0 0 180) (size 3.2 3.2) (drill 3.2) (layers "*.Cu" "*.Mask")))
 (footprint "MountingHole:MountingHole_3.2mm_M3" (layer "B.Cu") (at 160 97 180)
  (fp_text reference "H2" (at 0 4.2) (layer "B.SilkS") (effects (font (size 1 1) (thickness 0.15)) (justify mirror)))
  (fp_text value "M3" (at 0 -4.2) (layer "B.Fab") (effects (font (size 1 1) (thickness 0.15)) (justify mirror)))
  (pad "" np_thru_hole circle (at 0 0 180) (size 3.2 3.2) (drill 3.2) (layers "*.Cu" "*.Mask")))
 (gr_rect (start 138.5 93.5) (end 163.5 118.5) (stroke (width 0.1) (type default)) (fill none) (layer "Edge.Cuts"))
 (via (at 170.5 110) (size 0.6) (drill 0.3) (layers "F.Cu" "B.Cu") (free) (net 48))
 (via (at 170.5 110.75) (size 0.6) (drill 0.3) (layers "F.Cu" "B.Cu") (free) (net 48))
 (via (at 171.25 110) (size 0.6) (drill 0.3) (layers "F.Cu" "B.Cu") (free) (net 48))
 (via (at 171.25 110.75) (size 0.6) (drill 0.3) (layers "F.Cu" "B.Cu") (free) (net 48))
 (via (at 147.75 107) (size 0.6) (drill 0.3) (layers "F.Cu" "B.Cu") (free) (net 47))
 (via (at 148.5 107) (size 0.6) (drill 0.3) (layers "F.Cu" "B.Cu") (free) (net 47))
 (segment (start 128.75 102) (end 128.75 103.3325) (width 0.2) (layer "F.Cu") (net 3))
 (segment (start 129.75 102) (end 129.75 103.3325) (width 0.2) (layer "F.Cu") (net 3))
 (via (at 148 108.75) (size 0.6) (drill 0.3) (layers "F.Cu" "B.Cu") (free) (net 3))
 (via (at 134.75 107.5) (size 0.6) (drill 0.3) (layers "F.Cu" "B.Cu") (free) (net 3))
 (via (at 148 109.5) (size 0.6) (drill 0.3) (layers "F.Cu" "B.Cu") (free) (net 3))
 (via (at 135.5 107.5) (size 0.6) (drill 0.3) (layers "F.Cu" "B.Cu") (free) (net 3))
 (segment (start 169.02 106.27) (end 169 106.25) (width 0.2) (layer "F.Cu") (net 1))
 (segment (start 169.5 106.27) (end 169.02 106.27) (width 0.2) (layer "F.Cu") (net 1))
 (via (at 169 106.25) (size 0.6) (drill 0.3) (layers "F.Cu" "B.Cu") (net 1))
 (segment (start 169.56 106.25) (end 169 106.25) (width 0.2) (layer "B.Cu") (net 1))
 (segment (start 120.98 96.5625) (end 120.98 97.5325) (width 0.2) (layer "F.Cu") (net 49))
 (segment (start 125.25 102) (end 125.25 103.5625) (width 0.2) (layer "F.Cu") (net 16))
 (segment (start 125.75 102) (end 125.75 103.0625) (width 0.2) (layer "F.Cu") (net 17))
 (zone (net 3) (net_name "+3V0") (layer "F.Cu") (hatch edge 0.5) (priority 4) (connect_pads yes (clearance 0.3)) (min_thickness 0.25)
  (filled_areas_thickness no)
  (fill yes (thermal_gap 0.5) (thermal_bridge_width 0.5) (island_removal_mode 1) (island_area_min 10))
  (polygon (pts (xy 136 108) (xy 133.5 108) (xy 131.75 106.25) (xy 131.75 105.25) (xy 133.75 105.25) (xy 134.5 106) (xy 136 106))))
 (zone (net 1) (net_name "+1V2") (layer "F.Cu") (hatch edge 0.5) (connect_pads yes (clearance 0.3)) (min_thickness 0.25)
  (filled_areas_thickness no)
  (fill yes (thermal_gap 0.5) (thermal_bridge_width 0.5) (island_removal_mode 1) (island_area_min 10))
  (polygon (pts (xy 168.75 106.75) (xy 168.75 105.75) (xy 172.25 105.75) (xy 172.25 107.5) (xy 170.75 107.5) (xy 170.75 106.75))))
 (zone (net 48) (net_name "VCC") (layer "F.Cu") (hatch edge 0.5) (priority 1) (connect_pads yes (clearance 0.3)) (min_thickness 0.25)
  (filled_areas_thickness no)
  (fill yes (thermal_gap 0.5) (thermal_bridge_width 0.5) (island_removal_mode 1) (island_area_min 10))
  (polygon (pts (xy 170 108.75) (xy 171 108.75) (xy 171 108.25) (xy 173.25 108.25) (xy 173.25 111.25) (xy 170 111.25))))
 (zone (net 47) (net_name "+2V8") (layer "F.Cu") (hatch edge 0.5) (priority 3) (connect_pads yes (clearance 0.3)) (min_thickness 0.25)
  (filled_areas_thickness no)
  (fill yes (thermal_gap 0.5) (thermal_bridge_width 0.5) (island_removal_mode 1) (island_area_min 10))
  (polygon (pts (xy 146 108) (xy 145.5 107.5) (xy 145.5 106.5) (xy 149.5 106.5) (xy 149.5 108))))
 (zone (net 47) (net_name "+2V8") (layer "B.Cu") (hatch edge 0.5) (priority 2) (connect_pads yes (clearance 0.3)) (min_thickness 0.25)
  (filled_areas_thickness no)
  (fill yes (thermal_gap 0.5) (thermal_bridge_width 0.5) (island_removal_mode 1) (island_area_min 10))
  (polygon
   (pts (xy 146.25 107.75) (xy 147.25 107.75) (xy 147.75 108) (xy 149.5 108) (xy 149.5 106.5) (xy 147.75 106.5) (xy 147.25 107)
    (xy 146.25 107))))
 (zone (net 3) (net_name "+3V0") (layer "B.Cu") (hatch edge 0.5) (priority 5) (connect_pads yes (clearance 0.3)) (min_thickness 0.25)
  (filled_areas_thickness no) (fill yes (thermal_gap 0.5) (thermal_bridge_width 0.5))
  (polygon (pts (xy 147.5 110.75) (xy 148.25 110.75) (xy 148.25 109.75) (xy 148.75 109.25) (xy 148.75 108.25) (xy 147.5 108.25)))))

